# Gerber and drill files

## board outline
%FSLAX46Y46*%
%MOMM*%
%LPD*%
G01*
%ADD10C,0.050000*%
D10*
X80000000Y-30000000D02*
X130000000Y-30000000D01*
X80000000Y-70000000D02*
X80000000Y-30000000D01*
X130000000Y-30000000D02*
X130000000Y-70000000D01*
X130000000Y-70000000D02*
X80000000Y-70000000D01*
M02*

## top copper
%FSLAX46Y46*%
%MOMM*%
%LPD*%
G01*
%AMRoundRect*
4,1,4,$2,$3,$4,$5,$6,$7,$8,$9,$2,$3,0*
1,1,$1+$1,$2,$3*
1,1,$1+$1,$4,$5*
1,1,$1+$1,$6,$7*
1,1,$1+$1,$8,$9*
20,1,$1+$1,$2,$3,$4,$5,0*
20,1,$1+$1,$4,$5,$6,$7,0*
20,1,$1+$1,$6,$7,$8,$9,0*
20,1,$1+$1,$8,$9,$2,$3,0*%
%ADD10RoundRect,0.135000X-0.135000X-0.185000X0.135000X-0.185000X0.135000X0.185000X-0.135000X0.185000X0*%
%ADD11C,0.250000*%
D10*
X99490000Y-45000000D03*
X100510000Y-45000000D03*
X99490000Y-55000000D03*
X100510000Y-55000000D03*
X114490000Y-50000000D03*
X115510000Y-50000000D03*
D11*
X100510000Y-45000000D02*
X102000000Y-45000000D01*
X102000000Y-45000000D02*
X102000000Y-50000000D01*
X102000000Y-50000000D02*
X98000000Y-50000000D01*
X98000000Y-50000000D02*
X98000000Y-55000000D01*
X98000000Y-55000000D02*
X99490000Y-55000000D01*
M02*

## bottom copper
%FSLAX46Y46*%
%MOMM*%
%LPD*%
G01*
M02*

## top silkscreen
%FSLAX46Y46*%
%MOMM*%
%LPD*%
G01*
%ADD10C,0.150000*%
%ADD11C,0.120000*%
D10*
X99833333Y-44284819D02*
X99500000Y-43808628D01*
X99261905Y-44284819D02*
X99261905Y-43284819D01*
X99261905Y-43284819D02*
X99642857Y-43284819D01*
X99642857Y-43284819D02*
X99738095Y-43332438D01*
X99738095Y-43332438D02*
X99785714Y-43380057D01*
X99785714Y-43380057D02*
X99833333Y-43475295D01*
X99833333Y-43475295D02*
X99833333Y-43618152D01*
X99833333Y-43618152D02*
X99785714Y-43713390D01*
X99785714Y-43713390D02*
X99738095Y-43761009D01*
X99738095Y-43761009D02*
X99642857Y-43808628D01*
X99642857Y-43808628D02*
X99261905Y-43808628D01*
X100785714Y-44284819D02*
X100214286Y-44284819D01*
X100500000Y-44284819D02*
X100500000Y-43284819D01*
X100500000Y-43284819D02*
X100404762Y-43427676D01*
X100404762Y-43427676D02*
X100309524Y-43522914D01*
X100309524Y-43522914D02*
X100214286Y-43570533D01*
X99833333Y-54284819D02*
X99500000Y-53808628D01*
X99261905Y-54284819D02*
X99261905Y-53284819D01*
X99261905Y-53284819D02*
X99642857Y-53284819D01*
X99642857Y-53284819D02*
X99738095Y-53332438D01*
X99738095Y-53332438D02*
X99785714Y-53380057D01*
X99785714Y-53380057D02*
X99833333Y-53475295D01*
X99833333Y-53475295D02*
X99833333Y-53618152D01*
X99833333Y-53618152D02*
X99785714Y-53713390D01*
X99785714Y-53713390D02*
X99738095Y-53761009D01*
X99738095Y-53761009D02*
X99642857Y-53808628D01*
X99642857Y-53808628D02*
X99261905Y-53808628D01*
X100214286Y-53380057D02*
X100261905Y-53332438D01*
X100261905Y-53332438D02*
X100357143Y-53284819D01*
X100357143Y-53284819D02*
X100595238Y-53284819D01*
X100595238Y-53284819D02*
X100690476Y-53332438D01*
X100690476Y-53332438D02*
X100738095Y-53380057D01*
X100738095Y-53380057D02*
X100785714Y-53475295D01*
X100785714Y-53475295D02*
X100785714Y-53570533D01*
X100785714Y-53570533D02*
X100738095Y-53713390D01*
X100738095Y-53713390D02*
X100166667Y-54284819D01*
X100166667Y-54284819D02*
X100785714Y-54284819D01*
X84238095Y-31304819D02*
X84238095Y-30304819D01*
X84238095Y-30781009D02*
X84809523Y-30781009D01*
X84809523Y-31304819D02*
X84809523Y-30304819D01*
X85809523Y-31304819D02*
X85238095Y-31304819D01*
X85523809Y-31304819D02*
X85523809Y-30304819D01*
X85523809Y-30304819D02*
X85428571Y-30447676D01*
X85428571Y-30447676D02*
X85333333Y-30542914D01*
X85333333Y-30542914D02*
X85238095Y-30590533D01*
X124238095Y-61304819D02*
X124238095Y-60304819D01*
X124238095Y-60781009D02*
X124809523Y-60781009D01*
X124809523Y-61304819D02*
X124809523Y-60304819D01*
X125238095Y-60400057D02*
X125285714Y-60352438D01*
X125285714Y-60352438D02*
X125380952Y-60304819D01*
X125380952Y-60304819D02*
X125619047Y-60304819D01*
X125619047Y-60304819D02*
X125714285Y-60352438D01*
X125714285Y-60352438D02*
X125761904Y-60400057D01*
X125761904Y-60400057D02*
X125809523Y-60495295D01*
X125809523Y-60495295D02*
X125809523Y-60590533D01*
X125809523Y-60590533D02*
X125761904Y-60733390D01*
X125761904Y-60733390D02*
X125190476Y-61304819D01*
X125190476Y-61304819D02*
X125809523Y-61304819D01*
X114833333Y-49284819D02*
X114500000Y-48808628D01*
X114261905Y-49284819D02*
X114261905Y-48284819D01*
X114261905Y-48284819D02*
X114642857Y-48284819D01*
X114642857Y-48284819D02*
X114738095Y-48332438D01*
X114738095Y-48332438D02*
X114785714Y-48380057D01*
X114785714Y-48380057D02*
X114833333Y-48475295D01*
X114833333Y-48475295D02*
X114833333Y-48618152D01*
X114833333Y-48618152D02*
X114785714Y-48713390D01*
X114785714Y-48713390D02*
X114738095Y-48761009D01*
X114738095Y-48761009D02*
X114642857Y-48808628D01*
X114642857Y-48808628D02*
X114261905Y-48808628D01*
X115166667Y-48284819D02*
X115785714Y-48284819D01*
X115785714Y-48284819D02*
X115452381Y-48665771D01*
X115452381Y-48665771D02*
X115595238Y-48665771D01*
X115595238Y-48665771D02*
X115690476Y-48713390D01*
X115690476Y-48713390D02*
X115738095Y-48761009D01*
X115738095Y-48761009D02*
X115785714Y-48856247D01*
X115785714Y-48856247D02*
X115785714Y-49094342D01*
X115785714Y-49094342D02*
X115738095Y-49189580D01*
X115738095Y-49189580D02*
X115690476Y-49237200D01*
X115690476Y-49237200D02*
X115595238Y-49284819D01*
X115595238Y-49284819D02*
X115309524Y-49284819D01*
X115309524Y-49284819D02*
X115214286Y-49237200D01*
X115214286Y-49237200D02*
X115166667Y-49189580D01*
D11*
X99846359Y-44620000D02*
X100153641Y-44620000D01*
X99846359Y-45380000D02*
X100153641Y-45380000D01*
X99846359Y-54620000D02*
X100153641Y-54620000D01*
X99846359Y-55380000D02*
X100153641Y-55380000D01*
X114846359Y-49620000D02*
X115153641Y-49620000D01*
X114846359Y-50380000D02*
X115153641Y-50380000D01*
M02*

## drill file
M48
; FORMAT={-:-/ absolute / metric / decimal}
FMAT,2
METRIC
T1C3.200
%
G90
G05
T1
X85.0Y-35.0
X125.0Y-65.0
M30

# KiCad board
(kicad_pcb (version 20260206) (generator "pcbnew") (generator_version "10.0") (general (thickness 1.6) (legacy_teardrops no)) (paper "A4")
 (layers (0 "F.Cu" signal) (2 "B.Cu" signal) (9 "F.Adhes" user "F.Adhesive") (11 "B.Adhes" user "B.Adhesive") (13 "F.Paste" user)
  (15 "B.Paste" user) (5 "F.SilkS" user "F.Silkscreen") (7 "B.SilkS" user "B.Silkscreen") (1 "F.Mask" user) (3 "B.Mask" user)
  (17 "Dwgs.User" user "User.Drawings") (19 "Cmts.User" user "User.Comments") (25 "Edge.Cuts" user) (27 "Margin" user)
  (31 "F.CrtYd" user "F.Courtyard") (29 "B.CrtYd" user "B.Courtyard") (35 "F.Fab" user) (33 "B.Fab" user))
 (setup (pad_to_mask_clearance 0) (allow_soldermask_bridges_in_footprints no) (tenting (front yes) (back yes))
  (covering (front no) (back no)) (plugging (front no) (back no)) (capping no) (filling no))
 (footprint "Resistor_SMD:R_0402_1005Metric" (layer "F.Cu") (at 100 45)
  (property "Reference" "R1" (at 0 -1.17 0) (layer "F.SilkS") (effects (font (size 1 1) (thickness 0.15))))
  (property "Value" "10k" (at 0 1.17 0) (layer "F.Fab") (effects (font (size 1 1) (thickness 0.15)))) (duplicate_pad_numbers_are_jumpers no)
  (fp_line (start -0.153641 -0.38) (end 0.153641 -0.38) (stroke (width 0.12) (type solid)) (layer "F.SilkS"))
  (fp_line (start -0.153641 0.38) (end 0.153641 0.38) (stroke (width 0.12) (type solid)) (layer "F.SilkS"))
  (pad "1" smd roundrect (at -0.51 0) (size 0.54 0.64) (layers "F.Cu" "F.Mask" "F.Paste") (roundrect_rratio 0.25) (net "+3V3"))
  (pad "2" smd roundrect (at 0.51 0) (size 0.54 0.64) (layers "F.Cu" "F.Mask" "F.Paste") (roundrect_rratio 0.25) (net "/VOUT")))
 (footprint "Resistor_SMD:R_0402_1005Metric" (layer "F.Cu") (at 100 55)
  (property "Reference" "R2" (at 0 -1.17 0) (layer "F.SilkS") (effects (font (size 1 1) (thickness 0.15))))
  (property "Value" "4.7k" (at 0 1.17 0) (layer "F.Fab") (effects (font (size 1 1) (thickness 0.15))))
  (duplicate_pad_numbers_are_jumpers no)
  (fp_line (start -0.153641 -0.38) (end 0.153641 -0.38) (stroke (width 0.12) (type solid)) (layer "F.SilkS"))
  (fp_line (start -0.153641 0.38) (end 0.153641 0.38) (stroke (width 0.12) (type solid)) (layer "F.SilkS"))
  (pad "1" smd roundrect (at -0.51 0) (size 0.54 0.64) (layers "F.Cu" "F.Mask" "F.Paste") (roundrect_rratio 0.25) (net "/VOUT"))
  (pad "2" smd roundrect (at 0.51 0) (size 0.54 0.64) (layers "F.Cu" "F.Mask" "F.Paste") (roundrect_rratio 0.25) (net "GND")))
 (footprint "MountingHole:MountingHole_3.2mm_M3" (layer "F.Cu") (at 85 35)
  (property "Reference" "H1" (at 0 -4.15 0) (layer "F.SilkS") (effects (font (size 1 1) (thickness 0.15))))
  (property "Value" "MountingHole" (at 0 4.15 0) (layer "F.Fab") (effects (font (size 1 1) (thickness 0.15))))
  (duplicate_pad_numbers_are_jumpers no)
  (pad "" np_thru_hole circle (at 0 0) (size 3.2 3.2) (drill 3.2) (layers "*.Cu" "*.Mask")))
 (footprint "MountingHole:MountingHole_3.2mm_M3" (layer "F.Cu") (at 125 65)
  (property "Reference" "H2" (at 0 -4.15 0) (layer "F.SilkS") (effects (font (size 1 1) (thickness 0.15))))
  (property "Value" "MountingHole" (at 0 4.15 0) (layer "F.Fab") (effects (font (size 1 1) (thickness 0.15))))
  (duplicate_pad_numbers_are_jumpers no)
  (pad "" np_thru_hole circle (at 0 0) (size 3.2 3.2) (drill 3.2) (layers "*.Cu" "*.Mask")))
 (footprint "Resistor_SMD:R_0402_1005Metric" (layer "F.Cu") (at 115 50)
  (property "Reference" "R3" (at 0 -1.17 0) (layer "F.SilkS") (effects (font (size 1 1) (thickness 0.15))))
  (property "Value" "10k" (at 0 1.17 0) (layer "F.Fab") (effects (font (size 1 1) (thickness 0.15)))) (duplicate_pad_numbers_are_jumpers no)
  (fp_line (start -0.153641 -0.38) (end 0.153641 -0.38) (stroke (width 0.12) (type solid)) (layer "F.SilkS"))
  (fp_line (start -0.153641 0.38) (end 0.153641 0.38) (stroke (width 0.12) (type solid)) (layer "F.SilkS"))
  (pad "1" smd roundrect (at -0.51 0) (size 0.54 0.64) (layers "F.Cu" "F.Mask" "F.Paste") (roundrect_rratio 0.25)
   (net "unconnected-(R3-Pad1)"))
  (pad "2" smd roundrect (at 0.51 0) (size 0.54 0.64) (layers "F.Cu" "F.Mask" "F.Paste") (roundrect_rratio 0.25)
   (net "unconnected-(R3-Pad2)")))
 (gr_line (start 80 30) (end 130 30) (stroke (width 0.05) (type default)) (layer "Edge.Cuts"))
 (gr_line (start 80 70) (end 80 30) (stroke (width 0.05) (type default)) (layer "Edge.Cuts"))
 (gr_line (start 130 30) (end 130 70) (stroke (width 0.05) (type default)) (layer "Edge.Cuts"))
 (gr_line (start 130 70) (end 80 70) (stroke (width 0.05) (type default)) (layer "Edge.Cuts"))
 (segment (start 100.51 45) (end 102 45) (width 0.25) (layer "F.Cu") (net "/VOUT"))
 (segment (start 102 45) (end 102 50) (width 0.25) (layer "F.Cu") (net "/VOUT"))
 (segment (start 102 50) (end 98 50) (width 0.25) (layer "F.Cu") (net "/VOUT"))
 (segment (start 98 50) (end 98 55) (width 0.25) (layer "F.Cu") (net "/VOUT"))
 (segment (start 98 55) (end 99.49 55) (width 0.25) (layer "F.Cu") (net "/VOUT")))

